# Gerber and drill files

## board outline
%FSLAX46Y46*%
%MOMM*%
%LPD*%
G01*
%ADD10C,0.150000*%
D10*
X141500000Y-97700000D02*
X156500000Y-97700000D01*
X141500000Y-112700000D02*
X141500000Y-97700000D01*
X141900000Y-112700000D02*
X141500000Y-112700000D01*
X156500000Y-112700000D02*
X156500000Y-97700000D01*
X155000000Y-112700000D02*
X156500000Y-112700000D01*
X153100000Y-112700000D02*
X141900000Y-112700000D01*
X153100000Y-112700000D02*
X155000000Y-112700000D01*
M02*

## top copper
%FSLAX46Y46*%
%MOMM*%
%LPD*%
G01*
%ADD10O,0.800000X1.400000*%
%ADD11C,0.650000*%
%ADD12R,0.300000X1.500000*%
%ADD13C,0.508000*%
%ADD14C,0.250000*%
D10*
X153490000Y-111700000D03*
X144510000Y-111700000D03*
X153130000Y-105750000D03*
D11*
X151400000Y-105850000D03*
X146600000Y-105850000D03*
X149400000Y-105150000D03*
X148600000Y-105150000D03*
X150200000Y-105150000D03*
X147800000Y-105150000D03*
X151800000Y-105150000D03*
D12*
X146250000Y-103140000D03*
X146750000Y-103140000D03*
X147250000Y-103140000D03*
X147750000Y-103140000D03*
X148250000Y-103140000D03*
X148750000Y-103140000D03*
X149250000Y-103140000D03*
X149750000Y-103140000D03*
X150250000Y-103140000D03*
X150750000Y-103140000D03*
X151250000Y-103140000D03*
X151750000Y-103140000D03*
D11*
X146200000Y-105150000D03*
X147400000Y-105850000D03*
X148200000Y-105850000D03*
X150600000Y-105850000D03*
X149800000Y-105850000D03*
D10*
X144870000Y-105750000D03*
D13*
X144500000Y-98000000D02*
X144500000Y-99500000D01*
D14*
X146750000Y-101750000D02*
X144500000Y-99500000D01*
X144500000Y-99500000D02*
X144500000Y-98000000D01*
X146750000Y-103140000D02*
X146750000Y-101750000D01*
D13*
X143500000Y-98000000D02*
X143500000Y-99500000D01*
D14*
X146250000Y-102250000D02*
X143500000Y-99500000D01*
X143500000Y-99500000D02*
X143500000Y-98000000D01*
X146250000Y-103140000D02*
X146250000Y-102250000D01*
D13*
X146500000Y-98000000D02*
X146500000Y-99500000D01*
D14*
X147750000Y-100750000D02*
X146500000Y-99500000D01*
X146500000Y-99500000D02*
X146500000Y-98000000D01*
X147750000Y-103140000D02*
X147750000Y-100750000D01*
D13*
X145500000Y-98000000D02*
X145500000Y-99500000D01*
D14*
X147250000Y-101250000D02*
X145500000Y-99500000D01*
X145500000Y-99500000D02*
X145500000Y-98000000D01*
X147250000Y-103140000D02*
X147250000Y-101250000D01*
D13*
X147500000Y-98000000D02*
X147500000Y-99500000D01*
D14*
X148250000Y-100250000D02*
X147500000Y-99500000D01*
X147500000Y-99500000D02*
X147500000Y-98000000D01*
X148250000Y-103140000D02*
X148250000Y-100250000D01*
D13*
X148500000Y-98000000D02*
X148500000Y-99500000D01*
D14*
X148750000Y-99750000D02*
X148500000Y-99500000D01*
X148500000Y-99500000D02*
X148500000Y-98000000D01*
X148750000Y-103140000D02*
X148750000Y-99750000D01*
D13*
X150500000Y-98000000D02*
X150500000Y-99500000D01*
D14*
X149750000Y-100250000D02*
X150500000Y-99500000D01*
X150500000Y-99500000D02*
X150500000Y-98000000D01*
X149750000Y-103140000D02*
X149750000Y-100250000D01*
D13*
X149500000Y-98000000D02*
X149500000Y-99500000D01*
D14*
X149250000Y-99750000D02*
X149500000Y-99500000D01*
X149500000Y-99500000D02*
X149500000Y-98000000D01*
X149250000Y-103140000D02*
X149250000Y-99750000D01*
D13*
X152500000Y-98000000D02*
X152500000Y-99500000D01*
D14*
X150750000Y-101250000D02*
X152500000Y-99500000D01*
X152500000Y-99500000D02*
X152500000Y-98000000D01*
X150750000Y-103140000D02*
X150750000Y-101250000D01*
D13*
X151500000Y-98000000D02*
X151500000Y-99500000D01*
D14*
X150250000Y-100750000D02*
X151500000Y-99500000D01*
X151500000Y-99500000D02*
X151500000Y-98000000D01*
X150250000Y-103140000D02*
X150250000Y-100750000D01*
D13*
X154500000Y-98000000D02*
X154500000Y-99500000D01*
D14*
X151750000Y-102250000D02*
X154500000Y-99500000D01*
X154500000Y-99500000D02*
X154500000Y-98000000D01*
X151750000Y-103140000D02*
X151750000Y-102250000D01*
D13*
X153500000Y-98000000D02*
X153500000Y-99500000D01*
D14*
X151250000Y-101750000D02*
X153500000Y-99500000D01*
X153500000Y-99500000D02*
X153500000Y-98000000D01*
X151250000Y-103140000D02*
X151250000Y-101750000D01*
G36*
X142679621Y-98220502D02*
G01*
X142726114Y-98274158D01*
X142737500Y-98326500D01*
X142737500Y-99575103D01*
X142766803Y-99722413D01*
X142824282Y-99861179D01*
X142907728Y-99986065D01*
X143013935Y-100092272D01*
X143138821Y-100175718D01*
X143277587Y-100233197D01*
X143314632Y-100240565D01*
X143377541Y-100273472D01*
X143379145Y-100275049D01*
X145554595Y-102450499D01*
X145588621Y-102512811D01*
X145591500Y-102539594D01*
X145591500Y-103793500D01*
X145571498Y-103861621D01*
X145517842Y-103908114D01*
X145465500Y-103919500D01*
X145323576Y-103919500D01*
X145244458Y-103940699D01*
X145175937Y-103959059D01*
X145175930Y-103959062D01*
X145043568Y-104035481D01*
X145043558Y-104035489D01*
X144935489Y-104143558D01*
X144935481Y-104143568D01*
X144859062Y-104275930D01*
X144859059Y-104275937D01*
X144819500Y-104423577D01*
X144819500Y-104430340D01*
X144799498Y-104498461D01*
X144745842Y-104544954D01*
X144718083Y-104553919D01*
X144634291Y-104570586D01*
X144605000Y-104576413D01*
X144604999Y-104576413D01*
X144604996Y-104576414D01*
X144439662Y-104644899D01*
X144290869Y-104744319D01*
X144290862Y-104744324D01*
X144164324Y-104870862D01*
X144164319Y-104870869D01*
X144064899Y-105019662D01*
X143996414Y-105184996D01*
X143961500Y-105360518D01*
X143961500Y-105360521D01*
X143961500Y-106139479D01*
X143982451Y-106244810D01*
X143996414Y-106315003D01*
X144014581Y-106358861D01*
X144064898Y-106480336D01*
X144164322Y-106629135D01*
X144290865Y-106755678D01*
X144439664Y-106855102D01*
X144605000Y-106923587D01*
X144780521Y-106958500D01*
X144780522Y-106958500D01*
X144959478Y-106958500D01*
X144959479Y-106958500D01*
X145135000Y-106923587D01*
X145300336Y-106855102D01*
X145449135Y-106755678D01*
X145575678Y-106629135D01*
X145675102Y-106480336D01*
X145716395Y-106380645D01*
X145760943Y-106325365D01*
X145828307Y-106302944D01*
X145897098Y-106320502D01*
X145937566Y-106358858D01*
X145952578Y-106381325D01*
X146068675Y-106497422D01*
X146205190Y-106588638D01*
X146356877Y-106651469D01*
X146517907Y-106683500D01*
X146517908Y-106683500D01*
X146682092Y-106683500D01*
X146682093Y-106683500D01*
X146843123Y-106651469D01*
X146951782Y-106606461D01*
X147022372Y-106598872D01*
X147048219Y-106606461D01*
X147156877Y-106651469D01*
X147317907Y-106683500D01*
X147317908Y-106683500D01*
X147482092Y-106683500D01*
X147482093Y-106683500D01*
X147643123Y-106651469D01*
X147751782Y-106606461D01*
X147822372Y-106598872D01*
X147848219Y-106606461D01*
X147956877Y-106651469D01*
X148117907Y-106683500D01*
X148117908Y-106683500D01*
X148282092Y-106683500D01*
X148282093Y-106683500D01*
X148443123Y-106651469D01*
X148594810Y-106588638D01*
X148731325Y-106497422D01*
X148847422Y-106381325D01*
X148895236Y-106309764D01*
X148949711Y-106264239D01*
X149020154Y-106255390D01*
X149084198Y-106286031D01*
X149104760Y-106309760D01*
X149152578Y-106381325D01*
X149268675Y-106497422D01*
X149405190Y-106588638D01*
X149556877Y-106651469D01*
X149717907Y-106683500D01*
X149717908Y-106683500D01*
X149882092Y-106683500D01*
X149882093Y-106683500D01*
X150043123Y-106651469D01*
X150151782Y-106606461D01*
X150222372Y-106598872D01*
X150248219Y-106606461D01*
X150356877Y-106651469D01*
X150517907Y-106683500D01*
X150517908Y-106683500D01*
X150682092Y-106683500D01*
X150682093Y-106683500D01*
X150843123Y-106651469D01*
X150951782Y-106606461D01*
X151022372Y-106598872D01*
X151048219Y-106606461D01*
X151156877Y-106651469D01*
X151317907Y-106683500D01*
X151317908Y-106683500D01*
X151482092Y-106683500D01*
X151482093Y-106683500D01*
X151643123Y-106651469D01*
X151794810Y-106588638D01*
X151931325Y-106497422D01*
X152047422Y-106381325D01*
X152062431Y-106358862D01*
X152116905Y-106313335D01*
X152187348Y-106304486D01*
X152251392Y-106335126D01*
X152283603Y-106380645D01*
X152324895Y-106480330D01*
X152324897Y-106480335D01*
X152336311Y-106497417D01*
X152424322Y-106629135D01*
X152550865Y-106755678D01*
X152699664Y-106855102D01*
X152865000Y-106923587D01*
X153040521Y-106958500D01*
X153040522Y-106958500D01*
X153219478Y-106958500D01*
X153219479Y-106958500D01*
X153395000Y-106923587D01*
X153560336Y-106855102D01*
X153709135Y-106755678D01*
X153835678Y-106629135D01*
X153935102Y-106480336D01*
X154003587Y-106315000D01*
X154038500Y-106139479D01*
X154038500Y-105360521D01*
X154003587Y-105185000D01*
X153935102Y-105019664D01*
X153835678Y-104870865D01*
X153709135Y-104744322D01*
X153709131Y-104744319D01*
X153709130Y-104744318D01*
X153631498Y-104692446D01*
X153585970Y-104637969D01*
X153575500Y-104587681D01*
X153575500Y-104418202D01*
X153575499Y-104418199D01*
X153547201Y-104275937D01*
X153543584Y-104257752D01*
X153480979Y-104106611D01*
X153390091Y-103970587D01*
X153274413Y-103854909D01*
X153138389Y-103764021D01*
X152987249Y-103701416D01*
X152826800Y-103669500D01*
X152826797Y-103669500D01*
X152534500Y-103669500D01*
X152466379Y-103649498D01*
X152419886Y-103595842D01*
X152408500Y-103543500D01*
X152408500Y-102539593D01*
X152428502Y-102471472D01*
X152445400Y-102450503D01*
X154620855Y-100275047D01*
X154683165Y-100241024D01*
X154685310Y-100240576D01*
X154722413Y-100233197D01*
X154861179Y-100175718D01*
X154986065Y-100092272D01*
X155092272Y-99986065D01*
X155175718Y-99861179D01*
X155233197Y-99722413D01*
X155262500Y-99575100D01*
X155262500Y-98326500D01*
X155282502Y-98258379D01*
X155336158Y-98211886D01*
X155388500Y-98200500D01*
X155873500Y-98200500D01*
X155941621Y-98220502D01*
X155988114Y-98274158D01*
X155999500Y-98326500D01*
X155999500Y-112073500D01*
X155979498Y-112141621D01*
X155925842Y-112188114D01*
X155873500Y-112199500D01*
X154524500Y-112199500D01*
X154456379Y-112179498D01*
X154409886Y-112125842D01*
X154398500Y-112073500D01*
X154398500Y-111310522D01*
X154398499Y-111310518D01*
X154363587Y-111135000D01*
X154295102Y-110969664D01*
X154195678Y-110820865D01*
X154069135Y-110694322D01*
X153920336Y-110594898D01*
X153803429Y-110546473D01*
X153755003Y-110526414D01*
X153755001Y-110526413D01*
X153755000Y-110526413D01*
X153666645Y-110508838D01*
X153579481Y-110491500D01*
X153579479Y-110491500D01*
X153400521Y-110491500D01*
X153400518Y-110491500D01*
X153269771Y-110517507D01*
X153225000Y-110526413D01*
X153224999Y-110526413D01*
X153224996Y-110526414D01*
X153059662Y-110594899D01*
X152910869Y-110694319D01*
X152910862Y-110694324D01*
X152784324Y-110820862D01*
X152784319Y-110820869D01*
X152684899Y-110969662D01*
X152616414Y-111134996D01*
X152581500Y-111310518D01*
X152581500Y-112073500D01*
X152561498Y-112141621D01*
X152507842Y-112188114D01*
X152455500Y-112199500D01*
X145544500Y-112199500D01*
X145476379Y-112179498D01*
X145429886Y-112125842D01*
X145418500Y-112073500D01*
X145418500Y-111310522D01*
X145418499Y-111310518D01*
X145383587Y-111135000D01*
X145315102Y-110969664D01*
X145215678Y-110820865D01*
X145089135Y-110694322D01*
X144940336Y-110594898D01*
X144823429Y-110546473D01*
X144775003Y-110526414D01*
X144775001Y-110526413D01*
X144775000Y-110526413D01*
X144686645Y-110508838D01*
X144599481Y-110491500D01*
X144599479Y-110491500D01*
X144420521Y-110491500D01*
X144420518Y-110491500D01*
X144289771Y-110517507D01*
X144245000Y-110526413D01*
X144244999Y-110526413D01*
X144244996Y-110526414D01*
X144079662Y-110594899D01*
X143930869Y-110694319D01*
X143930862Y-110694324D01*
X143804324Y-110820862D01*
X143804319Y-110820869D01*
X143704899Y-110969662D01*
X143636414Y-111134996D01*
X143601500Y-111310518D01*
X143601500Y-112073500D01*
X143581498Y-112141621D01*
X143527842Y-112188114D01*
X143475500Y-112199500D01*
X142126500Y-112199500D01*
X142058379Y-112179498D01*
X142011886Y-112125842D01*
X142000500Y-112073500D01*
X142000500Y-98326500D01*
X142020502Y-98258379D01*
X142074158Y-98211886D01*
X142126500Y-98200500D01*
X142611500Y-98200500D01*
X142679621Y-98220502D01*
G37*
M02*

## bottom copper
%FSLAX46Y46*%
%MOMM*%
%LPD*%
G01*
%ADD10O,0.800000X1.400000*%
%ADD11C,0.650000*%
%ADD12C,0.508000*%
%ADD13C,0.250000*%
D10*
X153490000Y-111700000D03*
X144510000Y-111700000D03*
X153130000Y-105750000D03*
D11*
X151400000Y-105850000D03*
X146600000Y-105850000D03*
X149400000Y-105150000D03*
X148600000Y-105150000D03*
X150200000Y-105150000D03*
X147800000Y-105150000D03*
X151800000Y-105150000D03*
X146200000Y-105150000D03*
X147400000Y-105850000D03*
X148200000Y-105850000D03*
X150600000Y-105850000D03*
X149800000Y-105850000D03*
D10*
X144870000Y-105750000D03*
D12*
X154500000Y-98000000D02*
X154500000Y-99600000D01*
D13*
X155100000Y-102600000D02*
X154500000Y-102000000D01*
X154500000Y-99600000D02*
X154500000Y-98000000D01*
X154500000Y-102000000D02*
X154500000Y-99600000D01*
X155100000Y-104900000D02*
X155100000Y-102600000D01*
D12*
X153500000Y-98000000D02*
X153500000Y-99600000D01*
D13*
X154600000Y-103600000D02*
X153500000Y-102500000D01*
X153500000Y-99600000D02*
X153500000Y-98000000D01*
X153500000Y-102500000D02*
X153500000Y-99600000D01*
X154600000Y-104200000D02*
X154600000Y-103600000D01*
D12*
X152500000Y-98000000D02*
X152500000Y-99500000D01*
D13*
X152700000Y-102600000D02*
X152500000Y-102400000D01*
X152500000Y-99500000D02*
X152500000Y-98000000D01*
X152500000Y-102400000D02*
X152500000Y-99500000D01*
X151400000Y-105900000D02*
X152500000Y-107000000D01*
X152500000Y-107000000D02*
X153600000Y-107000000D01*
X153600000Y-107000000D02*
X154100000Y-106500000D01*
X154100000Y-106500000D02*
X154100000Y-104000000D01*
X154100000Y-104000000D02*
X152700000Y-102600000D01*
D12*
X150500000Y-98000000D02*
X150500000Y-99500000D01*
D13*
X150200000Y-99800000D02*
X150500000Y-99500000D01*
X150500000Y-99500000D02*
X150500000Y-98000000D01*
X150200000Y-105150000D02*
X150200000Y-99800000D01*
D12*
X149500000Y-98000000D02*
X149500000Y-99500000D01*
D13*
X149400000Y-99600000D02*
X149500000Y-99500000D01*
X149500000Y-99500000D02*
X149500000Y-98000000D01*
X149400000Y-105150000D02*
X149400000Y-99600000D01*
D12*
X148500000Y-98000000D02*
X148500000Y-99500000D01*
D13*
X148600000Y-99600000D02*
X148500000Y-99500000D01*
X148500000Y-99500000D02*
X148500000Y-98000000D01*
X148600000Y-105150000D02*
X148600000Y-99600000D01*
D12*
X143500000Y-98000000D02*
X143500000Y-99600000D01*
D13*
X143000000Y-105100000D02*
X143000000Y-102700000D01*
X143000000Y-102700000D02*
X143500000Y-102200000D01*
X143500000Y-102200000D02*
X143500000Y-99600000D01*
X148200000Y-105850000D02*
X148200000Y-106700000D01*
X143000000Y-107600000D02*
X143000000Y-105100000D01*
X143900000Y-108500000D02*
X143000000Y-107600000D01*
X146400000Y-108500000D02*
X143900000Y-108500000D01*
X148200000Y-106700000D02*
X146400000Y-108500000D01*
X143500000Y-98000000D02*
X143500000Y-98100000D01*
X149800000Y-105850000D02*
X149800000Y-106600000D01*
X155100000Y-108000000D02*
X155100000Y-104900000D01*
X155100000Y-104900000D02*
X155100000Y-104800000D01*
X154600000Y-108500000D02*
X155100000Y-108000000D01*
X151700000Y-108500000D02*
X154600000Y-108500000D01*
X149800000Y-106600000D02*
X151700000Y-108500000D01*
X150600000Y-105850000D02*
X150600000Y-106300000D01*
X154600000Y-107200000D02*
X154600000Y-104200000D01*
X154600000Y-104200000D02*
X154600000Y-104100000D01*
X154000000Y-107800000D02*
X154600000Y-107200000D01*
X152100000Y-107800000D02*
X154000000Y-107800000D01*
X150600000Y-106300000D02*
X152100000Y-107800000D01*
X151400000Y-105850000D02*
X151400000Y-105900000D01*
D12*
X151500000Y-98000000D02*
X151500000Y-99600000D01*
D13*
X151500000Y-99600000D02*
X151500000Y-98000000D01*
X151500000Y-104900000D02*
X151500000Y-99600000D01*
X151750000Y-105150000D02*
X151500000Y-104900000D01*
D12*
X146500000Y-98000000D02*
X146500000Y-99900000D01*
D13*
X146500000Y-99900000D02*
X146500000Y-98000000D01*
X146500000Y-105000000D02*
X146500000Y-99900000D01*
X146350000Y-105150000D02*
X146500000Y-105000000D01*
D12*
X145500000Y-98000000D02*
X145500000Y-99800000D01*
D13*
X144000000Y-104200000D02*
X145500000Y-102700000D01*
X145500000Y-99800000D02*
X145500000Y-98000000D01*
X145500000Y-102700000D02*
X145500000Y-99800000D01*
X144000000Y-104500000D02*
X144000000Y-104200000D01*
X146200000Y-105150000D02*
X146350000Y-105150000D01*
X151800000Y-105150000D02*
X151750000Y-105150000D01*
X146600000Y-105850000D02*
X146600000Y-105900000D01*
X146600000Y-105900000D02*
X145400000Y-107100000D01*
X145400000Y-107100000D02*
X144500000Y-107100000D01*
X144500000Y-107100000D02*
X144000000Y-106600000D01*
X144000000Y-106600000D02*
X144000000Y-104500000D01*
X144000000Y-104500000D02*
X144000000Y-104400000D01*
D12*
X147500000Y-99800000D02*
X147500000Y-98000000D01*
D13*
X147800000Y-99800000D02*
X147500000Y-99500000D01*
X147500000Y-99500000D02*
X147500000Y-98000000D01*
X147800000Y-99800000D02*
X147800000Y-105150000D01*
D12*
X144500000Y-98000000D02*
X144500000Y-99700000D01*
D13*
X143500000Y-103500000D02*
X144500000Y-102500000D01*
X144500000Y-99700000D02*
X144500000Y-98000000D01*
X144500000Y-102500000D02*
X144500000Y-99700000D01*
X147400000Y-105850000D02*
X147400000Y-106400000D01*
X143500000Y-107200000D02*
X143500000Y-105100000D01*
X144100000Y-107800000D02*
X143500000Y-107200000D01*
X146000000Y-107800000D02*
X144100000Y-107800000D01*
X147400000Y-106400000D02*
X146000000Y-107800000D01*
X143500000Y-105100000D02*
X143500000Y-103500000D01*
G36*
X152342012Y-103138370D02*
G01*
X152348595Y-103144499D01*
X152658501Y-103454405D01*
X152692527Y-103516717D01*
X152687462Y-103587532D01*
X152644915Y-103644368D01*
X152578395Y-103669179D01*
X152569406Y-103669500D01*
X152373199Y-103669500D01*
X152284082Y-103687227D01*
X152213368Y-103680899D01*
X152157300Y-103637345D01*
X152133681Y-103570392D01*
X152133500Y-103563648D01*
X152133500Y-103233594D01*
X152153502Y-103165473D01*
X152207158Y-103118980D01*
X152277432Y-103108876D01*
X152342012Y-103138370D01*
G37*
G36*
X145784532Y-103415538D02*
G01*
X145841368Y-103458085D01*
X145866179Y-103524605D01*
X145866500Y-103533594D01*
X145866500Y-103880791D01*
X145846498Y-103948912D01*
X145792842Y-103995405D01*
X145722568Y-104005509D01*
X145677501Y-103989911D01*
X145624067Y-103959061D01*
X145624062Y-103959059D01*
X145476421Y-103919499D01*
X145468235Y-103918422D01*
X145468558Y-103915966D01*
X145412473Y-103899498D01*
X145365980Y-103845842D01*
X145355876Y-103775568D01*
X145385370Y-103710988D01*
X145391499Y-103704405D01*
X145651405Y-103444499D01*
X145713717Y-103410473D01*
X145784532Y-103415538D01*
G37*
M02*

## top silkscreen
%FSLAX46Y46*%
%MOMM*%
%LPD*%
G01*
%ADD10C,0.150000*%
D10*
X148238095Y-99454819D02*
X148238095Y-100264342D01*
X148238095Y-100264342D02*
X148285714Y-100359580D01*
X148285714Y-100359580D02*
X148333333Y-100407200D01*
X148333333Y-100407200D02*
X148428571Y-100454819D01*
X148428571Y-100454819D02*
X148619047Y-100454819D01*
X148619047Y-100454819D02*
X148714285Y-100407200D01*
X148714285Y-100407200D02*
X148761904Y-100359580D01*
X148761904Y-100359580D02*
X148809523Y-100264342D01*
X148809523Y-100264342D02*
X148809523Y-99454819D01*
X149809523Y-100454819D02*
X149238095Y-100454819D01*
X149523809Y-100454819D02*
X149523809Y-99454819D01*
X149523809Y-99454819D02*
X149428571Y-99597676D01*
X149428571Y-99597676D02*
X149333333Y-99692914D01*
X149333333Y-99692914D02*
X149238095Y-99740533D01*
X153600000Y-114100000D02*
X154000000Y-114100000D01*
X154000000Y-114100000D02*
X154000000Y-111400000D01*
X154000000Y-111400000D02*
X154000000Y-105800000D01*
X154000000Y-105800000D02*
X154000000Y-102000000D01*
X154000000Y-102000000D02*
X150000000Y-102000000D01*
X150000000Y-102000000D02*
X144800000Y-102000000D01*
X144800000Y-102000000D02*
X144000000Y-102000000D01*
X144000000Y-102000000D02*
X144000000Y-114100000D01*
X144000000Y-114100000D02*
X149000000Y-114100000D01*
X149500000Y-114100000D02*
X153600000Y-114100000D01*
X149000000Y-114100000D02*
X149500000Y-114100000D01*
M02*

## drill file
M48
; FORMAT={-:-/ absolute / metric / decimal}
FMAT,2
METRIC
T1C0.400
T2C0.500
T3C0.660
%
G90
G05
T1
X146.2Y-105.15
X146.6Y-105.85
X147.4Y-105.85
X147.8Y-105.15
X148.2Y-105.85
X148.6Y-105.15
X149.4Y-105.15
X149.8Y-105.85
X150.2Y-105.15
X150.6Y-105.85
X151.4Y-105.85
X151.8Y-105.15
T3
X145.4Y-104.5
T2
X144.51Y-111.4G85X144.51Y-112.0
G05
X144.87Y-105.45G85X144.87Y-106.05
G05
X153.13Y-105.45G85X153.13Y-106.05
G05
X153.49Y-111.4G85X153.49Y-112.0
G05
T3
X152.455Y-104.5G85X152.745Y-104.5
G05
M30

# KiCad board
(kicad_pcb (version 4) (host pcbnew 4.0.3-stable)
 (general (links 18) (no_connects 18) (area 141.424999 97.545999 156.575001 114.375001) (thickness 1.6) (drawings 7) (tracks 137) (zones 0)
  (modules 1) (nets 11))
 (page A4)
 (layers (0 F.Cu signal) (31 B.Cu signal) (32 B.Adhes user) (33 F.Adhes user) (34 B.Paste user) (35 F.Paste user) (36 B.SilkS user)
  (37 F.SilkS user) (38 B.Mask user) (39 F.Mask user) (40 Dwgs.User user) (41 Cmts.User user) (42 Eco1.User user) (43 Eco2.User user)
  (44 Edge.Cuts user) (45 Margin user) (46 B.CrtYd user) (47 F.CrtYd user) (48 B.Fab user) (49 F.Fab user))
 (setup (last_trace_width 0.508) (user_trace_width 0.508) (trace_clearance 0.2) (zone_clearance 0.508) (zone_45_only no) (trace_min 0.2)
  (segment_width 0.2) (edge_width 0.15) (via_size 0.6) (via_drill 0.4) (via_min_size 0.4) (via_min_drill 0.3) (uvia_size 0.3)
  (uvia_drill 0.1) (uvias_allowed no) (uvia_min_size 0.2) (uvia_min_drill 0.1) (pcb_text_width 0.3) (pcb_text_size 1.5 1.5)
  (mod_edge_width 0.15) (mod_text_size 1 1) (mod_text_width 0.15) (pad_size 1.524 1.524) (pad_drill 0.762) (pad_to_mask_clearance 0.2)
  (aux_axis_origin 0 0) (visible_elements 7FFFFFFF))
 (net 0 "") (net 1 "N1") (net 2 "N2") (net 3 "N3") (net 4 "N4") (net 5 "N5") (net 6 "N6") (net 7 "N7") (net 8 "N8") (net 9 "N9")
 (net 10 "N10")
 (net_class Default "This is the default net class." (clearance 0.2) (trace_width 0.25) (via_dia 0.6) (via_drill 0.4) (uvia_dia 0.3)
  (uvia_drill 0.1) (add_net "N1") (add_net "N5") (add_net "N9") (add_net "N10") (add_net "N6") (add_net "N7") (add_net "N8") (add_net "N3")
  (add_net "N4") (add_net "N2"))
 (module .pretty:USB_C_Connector (layer F.Cu) (at 149 104.5)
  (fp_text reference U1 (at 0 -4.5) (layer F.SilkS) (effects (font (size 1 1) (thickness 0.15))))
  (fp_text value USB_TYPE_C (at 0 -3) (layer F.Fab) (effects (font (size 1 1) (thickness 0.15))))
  (fp_line (start 4.6 9.6) (end 5 9.6) (layer F.SilkS) (width 0.15))
  (fp_line (start 5 9.6) (end 5 6.9) (layer F.SilkS) (width 0.15))
  (fp_line (start 5 6.9) (end 5 1.3) (layer F.SilkS) (width 0.15))
  (fp_line (start 5 1.3) (end 5 -2.5) (layer F.SilkS) (width 0.15))
  (fp_line (start 5 -2.5) (end 1 -2.5) (layer F.SilkS) (width 0.15))
  (fp_line (start 1 -2.5) (end -4.2 -2.5) (layer F.SilkS) (width 0.15))
  (fp_line (start -4.2 -2.5) (end -5 -2.5) (layer F.SilkS) (width 0.15))
  (fp_line (start -5 -2.5) (end -5 9.6) (layer F.SilkS) (width 0.15))
  (fp_line (start -5 9.6) (end 0 9.6) (layer F.SilkS) (width 0.15))
  (fp_line (start 0.5 9.6) (end 4.6 9.6) (layer F.SilkS) (width 0.15))
  (fp_line (start 0 9.6) (end 0.5 9.6) (layer F.SilkS) (width 0.15))
  (pad 0 thru_hole oval (at 4.49 7.2) (size 0.8 1.4) (drill oval 0.5 1.1) (layers *.Cu *.Mask) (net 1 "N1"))
  (pad 0 thru_hole oval (at -4.49 7.2) (size 0.8 1.4) (drill oval 0.5 1.1) (layers *.Cu *.Mask) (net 1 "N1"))
  (pad 0 thru_hole oval (at 4.13 1.25) (size 0.8 1.4) (drill oval 0.5 1.1) (layers *.Cu *.Mask) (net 1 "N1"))
  (pad "" np_thru_hole oval (at 3.6 0) (size 0.95 0.66) (drill oval 0.95 0.66) (layers *.Cu *.Mask))
  (pad B2 thru_hole circle (at 2.4 1.35) (size 0.65 0.65) (drill 0.4) (layers *.Cu *.Mask) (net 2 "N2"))
  (pad B11 thru_hole circle (at -2.4 1.35) (size 0.65 0.65) (drill 0.4) (layers *.Cu *.Mask) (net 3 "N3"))
  (pad B6 thru_hole circle (at 0.4 0.65) (size 0.65 0.65) (drill 0.4) (layers *.Cu *.Mask) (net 2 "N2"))
  (pad B7 thru_hole circle (at -0.4 0.65) (size 0.65 0.65) (drill 0.4) (layers *.Cu *.Mask) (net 2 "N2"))
  (pad B4 thru_hole circle (at 1.2 0.65) (size 0.65 0.65) (drill 0.4) (layers *.Cu *.Mask) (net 2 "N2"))
  (pad B9 thru_hole circle (at -1.2 0.65) (size 0.65 0.65) (drill 0.4) (layers *.Cu *.Mask) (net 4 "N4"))
  (pad B1 thru_hole circle (at 2.8 0.65) (size 0.65 0.65) (drill 0.4) (layers *.Cu *.Mask) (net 3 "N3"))
  (pad A1 smd rect (at -2.75 -1.36) (size 0.3 1.5) (layers F.Cu F.Paste F.Mask) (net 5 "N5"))
  (pad A2 smd rect (at -2.25 -1.36) (size 0.3 1.5) (layers F.Cu F.Paste F.Mask) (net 5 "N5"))
  (pad A3 smd rect (at -1.75 -1.36) (size 0.3 1.5) (layers F.Cu F.Paste F.Mask) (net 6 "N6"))
  (pad A4 smd rect (at -1.25 -1.36) (size 0.3 1.5) (layers F.Cu F.Paste F.Mask) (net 6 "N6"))
  (pad A5 smd rect (at -0.75 -1.36) (size 0.3 1.5) (layers F.Cu F.Paste F.Mask) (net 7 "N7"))
  (pad A6 smd rect (at -0.25 -1.36) (size 0.3 1.5) (layers F.Cu F.Paste F.Mask) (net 7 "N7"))
  (pad A7 smd rect (at 0.25 -1.36) (size 0.3 1.5) (layers F.Cu F.Paste F.Mask) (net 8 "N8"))
  (pad A8 smd rect (at 0.75 -1.36) (size 0.3 1.5) (layers F.Cu F.Paste F.Mask) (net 8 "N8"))
  (pad A9 smd rect (at 1.25 -1.36) (size 0.3 1.5) (layers F.Cu F.Paste F.Mask) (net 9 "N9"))
  (pad A10 smd rect (at 1.75 -1.36) (size 0.3 1.5) (layers F.Cu F.Paste F.Mask) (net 9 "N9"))
  (pad A11 smd rect (at 2.25 -1.36) (size 0.3 1.5) (layers F.Cu F.Paste F.Mask) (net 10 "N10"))
  (pad A12 smd rect (at 2.75 -1.36) (size 0.3 1.5) (layers F.Cu F.Paste F.Mask) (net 10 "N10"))
  (pad B12 thru_hole circle (at -2.8 0.65) (size 0.65 0.65) (drill 0.4) (layers *.Cu *.Mask) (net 3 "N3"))
  (pad B10 thru_hole circle (at -1.6 1.35) (size 0.65 0.65) (drill 0.4) (layers *.Cu *.Mask) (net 4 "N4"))
  (pad B8 thru_hole circle (at -0.8 1.35) (size 0.65 0.65) (drill 0.4) (layers *.Cu *.Mask) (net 2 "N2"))
  (pad B3 thru_hole circle (at 1.6 1.35) (size 0.65 0.65) (drill 0.4) (layers *.Cu *.Mask) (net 2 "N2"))
  (pad B5 thru_hole circle (at 0.8 1.35) (size 0.65 0.65) (drill 0.4) (layers *.Cu *.Mask) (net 2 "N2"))
  (pad "" np_thru_hole circle (at -3.6 0) (size 0.66 0.66) (drill 0.66) (layers *.Cu *.Mask))
  (pad 0 thru_hole oval (at -4.13 1.25) (size 0.8 1.4) (drill oval 0.5 1.1) (layers *.Cu *.Mask) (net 1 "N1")))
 (gr_line (start 141.5 97.7) (end 156.5 97.7) (angle 90) (layer Edge.Cuts) (width 0.15))
 (gr_line (start 141.5 112.7) (end 141.5 97.7) (angle 90) (layer Edge.Cuts) (width 0.15))
 (gr_line (start 141.9 112.7) (end 141.5 112.7) (angle 90) (layer Edge.Cuts) (width 0.15))
 (gr_line (start 156.5 112.7) (end 156.5 97.7) (angle 90) (layer Edge.Cuts) (width 0.15))
 (gr_line (start 155 112.7) (end 156.5 112.7) (angle 90) (layer Edge.Cuts) (width 0.15))
 (gr_line (start 153.1 112.7) (end 141.9 112.7) (angle 90) (layer Edge.Cuts) (width 0.15))
 (gr_line (start 153.1 112.7) (end 155 112.7) (angle 90) (layer Edge.Cuts) (width 0.15))
 (segment (start 154.5 98) (end 154.5 99.6) (width 0.508) (layer B.Cu) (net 2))
 (segment (start 155.1 102.6) (end 154.5 102) (width 0.25) (layer B.Cu) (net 2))
 (segment (start 154.5 99.6) (end 154.5 98) (width 0.25) (layer B.Cu) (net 2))
 (segment (start 154.5 102) (end 154.5 99.6) (width 0.25) (layer B.Cu) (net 2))
 (segment (start 155.1 104.9) (end 155.1 102.6) (width 0.25) (layer B.Cu) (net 2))
 (segment (start 153.5 98) (end 153.5 99.6) (width 0.508) (layer B.Cu) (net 2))
 (segment (start 154.6 103.6) (end 153.5 102.5) (width 0.25) (layer B.Cu) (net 2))
 (segment (start 153.5 99.6) (end 153.5 98) (width 0.25) (layer B.Cu) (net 2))
 (segment (start 153.5 102.5) (end 153.5 99.6) (width 0.25) (layer B.Cu) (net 2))
 (segment (start 154.6 104.2) (end 154.6 103.6) (width 0.25) (layer B.Cu) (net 2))
 (segment (start 152.5 98) (end 152.5 99.5) (width 0.508) (layer B.Cu) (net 2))
 (segment (start 152.7 102.6) (end 152.5 102.4) (width 0.25) (layer B.Cu) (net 2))
 (segment (start 152.5 99.5) (end 152.5 98) (width 0.25) (layer B.Cu) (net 2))
 (segment (start 152.5 102.4) (end 152.5 99.5) (width 0.25) (layer B.Cu) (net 2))
 (segment (start 151.4 105.9) (end 152.5 107) (width 0.25) (layer B.Cu) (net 2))
 (segment (start 152.5 107) (end 153.6 107) (width 0.25) (layer B.Cu) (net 2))
 (segment (start 153.6 107) (end 154.1 106.5) (width 0.25) (layer B.Cu) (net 2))
 (segment (start 154.1 106.5) (end 154.1 104) (width 0.25) (layer B.Cu) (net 2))
 (segment (start 154.1 104) (end 152.7 102.6) (width 0.25) (layer B.Cu) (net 2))
 (segment (start 150.5 98) (end 150.5 99.5) (width 0.508) (layer B.Cu) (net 2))
 (segment (start 150.2 99.8) (end 150.5 99.5) (width 0.25) (layer B.Cu) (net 2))
 (segment (start 150.5 99.5) (end 150.5 98) (width 0.25) (layer B.Cu) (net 2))
 (segment (start 150.2 105.15) (end 150.2 99.8) (width 0.25) (layer B.Cu) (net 2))
 (segment (start 149.5 98) (end 149.5 99.5) (width 0.508) (layer B.Cu) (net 2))
 (segment (start 149.4 99.6) (end 149.5 99.5) (width 0.25) (layer B.Cu) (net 2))
 (segment (start 149.5 99.5) (end 149.5 98) (width 0.25) (layer B.Cu) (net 2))
 (segment (start 149.4 105.15) (end 149.4 99.6) (width 0.25) (layer B.Cu) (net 2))
 (segment (start 148.5 98) (end 148.5 99.5) (width 0.508) (layer B.Cu) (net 2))
 (segment (start 148.6 99.6) (end 148.5 99.5) (width 0.25) (layer B.Cu) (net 2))
 (segment (start 148.5 99.5) (end 148.5 98) (width 0.25) (layer B.Cu) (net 2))
 (segment (start 148.6 105.15) (end 148.6 99.6) (width 0.25) (layer B.Cu) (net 2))
 (segment (start 143.5 98) (end 143.5 99.6) (width 0.508) (layer B.Cu) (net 2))
 (segment (start 143 105.1) (end 143 102.7) (width 0.25) (layer B.Cu) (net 2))
 (segment (start 143 102.7) (end 143.5 102.2) (width 0.25) (layer B.Cu) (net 2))
 (segment (start 143.5 102.2) (end 143.5 99.6) (width 0.25) (layer B.Cu) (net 2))
 (segment (start 148.2 105.85) (end 148.2 106.7) (width 0.25) (layer B.Cu) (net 2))
 (segment (start 143 107.6) (end 143 105.1) (width 0.25) (layer B.Cu) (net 2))
 (segment (start 143.9 108.5) (end 143 107.6) (width 0.25) (layer B.Cu) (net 2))
 (segment (start 146.4 108.5) (end 143.9 108.5) (width 0.25) (layer B.Cu) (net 2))
 (segment (start 148.2 106.7) (end 146.4 108.5) (width 0.25) (layer B.Cu) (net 2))
 (segment (start 143.5 98) (end 143.5 98.1) (width 0.25) (layer B.Cu) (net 2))
 (segment (start 149.8 105.85) (end 149.8 106.6) (width 0.25) (layer B.Cu) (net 2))
 (segment (start 155.1 108) (end 155.1 104.9) (width 0.25) (layer B.Cu) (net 2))
 (segment (start 155.1 104.9) (end 155.1 104.8) (width 0.25) (layer B.Cu) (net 2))
 (segment (start 154.6 108.5) (end 155.1 108) (width 0.25) (layer B.Cu) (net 2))
 (segment (start 151.7 108.5) (end 154.6 108.5) (width 0.25) (layer B.Cu) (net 2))
 (segment (start 149.8 106.6) (end 151.7 108.5) (width 0.25) (layer B.Cu) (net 2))
 (segment (start 150.6 105.85) (end 150.6 106.3) (width 0.25) (layer B.Cu) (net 2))
 (segment (start 154.6 107.2) (end 154.6 104.2) (width 0.25) (layer B.Cu) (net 2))
 (segment (start 154.6 104.2) (end 154.6 104.1) (width 0.25) (layer B.Cu) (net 2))
 (segment (start 154 107.8) (end 154.6 107.2) (width 0.25) (layer B.Cu) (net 2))
 (segment (start 152.1 107.8) (end 154 107.8) (width 0.25) (layer B.Cu) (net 2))
 (segment (start 150.6 106.3) (end 152.1 107.8) (width 0.25) (layer B.Cu) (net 2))
 (segment (start 151.4 105.85) (end 151.4 105.9) (width 0.25) (layer B.Cu) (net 2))
 (segment (start 151.5 98) (end 151.5 99.6) (width 0.508) (layer B.Cu) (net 3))
 (segment (start 151.5 99.6) (end 151.5 98) (width 0.25) (layer B.Cu) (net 3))
 (segment (start 151.5 104.9) (end 151.5 99.6) (width 0.25) (layer B.Cu) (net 3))
 (segment (start 151.75 105.15) (end 151.5 104.9) (width 0.25) (layer B.Cu) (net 3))
 (segment (start 146.5 98) (end 146.5 99.9) (width 0.508) (layer B.Cu) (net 3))
 (segment (start 146.5 99.9) (end 146.5 98) (width 0.25) (layer B.Cu) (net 3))
 (segment (start 146.5 105) (end 146.5 99.9) (width 0.25) (layer B.Cu) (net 3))
 (segment (start 146.35 105.15) (end 146.5 105) (width 0.25) (layer B.Cu) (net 3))
 (segment (start 145.5 98) (end 145.5 99.8) (width 0.508) (layer B.Cu) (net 3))
 (segment (start 144 104.2) (end 145.5 102.7) (width 0.25) (layer B.Cu) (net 3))
 (segment (start 145.5 99.8) (end 145.5 98) (width 0.25) (layer B.Cu) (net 3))
 (segment (start 145.5 102.7) (end 145.5 99.8) (width 0.25) (layer B.Cu) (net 3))
 (segment (start 144 104.5) (end 144 104.2) (width 0.25) (layer B.Cu) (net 3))
 (segment (start 146.2 105.15) (end 146.35 105.15) (width 0.25) (layer B.Cu) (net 3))
 (segment (start 151.8 105.15) (end 151.75 105.15) (width 0.25) (layer B.Cu) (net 3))
 (segment (start 146.6 105.85) (end 146.6 105.9) (width 0.25) (layer B.Cu) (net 3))
 (segment (start 146.6 105.9) (end 145.4 107.1) (width 0.25) (layer B.Cu) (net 3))
 (segment (start 145.4 107.1) (end 144.5 107.1) (width 0.25) (layer B.Cu) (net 3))
 (segment (start 144.5 107.1) (end 144 106.6) (width 0.25) (layer B.Cu) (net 3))
 (segment (start 144 106.6) (end 144 104.5) (width 0.25) (layer B.Cu) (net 3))
 (segment (start 144 104.5) (end 144 104.4) (width 0.25) (layer B.Cu) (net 3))
 (segment (start 147.5 99.8) (end 147.5 98) (width 0.508) (layer B.Cu) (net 4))
 (segment (start 147.8 99.8) (end 147.5 99.5) (width 0.25) (layer B.Cu) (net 4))
 (segment (start 147.5 99.5) (end 147.5 98) (width 0.25) (layer B.Cu) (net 4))
 (segment (start 147.8 99.8) (end 147.8 105.15) (width 0.25) (layer B.Cu) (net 4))
 (segment (start 144.5 98) (end 144.5 99.7) (width 0.508) (layer B.Cu) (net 4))
 (segment (start 143.5 103.5) (end 144.5 102.5) (width 0.25) (layer B.Cu) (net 4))
 (segment (start 144.5 99.7) (end 144.5 98) (width 0.25) (layer B.Cu) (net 4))
 (segment (start 144.5 102.5) (end 144.5 99.7) (width 0.25) (layer B.Cu) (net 4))
 (segment (start 147.4 105.85) (end 147.4 106.4) (width 0.25) (layer B.Cu) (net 4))
 (segment (start 143.5 107.2) (end 143.5 105.1) (width 0.25) (layer B.Cu) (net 4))
 (segment (start 144.1 107.8) (end 143.5 107.2) (width 0.25) (layer B.Cu) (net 4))
 (segment (start 146 107.8) (end 144.1 107.8) (width 0.25) (layer B.Cu) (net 4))
 (segment (start 147.4 106.4) (end 146 107.8) (width 0.25) (layer B.Cu) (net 4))
 (segment (start 143.5 105.1) (end 143.5 103.5) (width 0.25) (layer B.Cu) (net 4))
 (segment (start 144.5 98) (end 144.5 99.5) (width 0.508) (layer F.Cu) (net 5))
 (segment (start 146.75 101.75) (end 144.5 99.5) (width 0.25) (layer F.Cu) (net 5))
 (segment (start 144.5 99.5) (end 144.5 98) (width 0.25) (layer F.Cu) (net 5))
 (segment (start 146.75 103.14) (end 146.75 101.75) (width 0.25) (layer F.Cu) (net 5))
 (segment (start 143.5 98) (end 143.5 99.5) (width 0.508) (layer F.Cu) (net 5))
 (segment (start 146.25 102.25) (end 143.5 99.5) (width 0.25) (layer F.Cu) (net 5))
 (segment (start 143.5 99.5) (end 143.5 98) (width 0.25) (layer F.Cu) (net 5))
 (segment (start 146.25 103.14) (end 146.25 102.25) (width 0.25) (layer F.Cu) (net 5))
 (segment (start 146.5 98) (end 146.5 99.5) (width 0.508) (layer F.Cu) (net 6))
 (segment (start 147.75 100.75) (end 146.5 99.5) (width 0.25) (layer F.Cu) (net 6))
 (segment (start 146.5 99.5) (end 146.5 98) (width 0.25) (layer F.Cu) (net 6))
 (segment (start 147.75 103.14) (end 147.75 100.75) (width 0.25) (layer F.Cu) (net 6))
 (segment (start 145.5 98) (end 145.5 99.5) (width 0.508) (layer F.Cu) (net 6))
 (segment (start 147.25 101.25) (end 145.5 99.5) (width 0.25) (layer F.Cu) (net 6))
 (segment (start 145.5 99.5) (end 145.5 98) (width 0.25) (layer F.Cu) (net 6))
 (segment (start 147.25 103.14) (end 147.25 101.25) (width 0.25) (layer F.Cu) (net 6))
 (segment (start 147.5 98) (end 147.5 99.5) (width 0.508) (layer F.Cu) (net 7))
 (segment (start 148.25 100.25) (end 147.5 99.5) (width 0.25) (layer F.Cu) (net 7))
 (segment (start 147.5 99.5) (end 147.5 98) (width 0.25) (layer F.Cu) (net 7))
 (segment (start 148.25 103.14) (end 148.25 100.25) (width 0.25) (layer F.Cu) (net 7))
 (segment (start 148.5 98) (end 148.5 99.5) (width 0.508) (layer F.Cu) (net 7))
 (segment (start 148.75 99.75) (end 148.5 99.5) (width 0.25) (layer F.Cu) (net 7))
 (segment (start 148.5 99.5) (end 148.5 98) (width 0.25) (layer F.Cu) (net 7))
 (segment (start 148.75 103.14) (end 148.75 99.75) (width 0.25) (layer F.Cu) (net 7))
 (segment (start 150.5 98) (end 150.5 99.5) (width 0.508) (layer F.Cu) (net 8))
 (segment (start 149.75 100.25) (end 150.5 99.5) (width 0.25) (layer F.Cu) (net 8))
 (segment (start 150.5 99.5) (end 150.5 98) (width 0.25) (layer F.Cu) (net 8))
 (segment (start 149.75 103.14) (end 149.75 100.25) (width 0.25) (layer F.Cu) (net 8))
 (segment (start 149.5 98) (end 149.5 99.5) (width 0.508) (layer F.Cu) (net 8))
 (segment (start 149.25 99.75) (end 149.5 99.5) (width 0.25) (layer F.Cu) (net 8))
 (segment (start 149.5 99.5) (end 149.5 98) (width 0.25) (layer F.Cu) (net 8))
 (segment (start 149.25 103.14) (end 149.25 99.75) (width 0.25) (layer F.Cu) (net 8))
 (segment (start 152.5 98) (end 152.5 99.5) (width 0.508) (layer F.Cu) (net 9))
 (segment (start 150.75 101.25) (end 152.5 99.5) (width 0.25) (layer F.Cu) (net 9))
 (segment (start 152.5 99.5) (end 152.5 98) (width 0.25) (layer F.Cu) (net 9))
 (segment (start 150.75 103.14) (end 150.75 101.25) (width 0.25) (layer F.Cu) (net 9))
 (segment (start 151.5 98) (end 151.5 99.5) (width 0.508) (layer F.Cu) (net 9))
 (segment (start 150.25 100.75) (end 151.5 99.5) (width 0.25) (layer F.Cu) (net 9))
 (segment (start 151.5 99.5) (end 151.5 98) (width 0.25) (layer F.Cu) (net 9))
 (segment (start 150.25 103.14) (end 150.25 100.75) (width 0.25) (layer F.Cu) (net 9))
 (segment (start 154.5 98) (end 154.5 99.5) (width 0.508) (layer F.Cu) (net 10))
 (segment (start 151.75 102.25) (end 154.5 99.5) (width 0.25) (layer F.Cu) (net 10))
 (segment (start 154.5 99.5) (end 154.5 98) (width 0.25) (layer F.Cu) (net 10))
 (segment (start 151.75 103.14) (end 151.75 102.25) (width 0.25) (layer F.Cu) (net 10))
 (segment (start 153.5 98) (end 153.5 99.5) (width 0.508) (layer F.Cu) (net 10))
 (segment (start 151.25 101.75) (end 153.5 99.5) (width 0.25) (layer F.Cu) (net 10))
 (segment (start 153.5 99.5) (end 153.5 98) (width 0.25) (layer F.Cu) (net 10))
 (segment (start 151.25 103.14) (end 151.25 101.75) (width 0.25) (layer F.Cu) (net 10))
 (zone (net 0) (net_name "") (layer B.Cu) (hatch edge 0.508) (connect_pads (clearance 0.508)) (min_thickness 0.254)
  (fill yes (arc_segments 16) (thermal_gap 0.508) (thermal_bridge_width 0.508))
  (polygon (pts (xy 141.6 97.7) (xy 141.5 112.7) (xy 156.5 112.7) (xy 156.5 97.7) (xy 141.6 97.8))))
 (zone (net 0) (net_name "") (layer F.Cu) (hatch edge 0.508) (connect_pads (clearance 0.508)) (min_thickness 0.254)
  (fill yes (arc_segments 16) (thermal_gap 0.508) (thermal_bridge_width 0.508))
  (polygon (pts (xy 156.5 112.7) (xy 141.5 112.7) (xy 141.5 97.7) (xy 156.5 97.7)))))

